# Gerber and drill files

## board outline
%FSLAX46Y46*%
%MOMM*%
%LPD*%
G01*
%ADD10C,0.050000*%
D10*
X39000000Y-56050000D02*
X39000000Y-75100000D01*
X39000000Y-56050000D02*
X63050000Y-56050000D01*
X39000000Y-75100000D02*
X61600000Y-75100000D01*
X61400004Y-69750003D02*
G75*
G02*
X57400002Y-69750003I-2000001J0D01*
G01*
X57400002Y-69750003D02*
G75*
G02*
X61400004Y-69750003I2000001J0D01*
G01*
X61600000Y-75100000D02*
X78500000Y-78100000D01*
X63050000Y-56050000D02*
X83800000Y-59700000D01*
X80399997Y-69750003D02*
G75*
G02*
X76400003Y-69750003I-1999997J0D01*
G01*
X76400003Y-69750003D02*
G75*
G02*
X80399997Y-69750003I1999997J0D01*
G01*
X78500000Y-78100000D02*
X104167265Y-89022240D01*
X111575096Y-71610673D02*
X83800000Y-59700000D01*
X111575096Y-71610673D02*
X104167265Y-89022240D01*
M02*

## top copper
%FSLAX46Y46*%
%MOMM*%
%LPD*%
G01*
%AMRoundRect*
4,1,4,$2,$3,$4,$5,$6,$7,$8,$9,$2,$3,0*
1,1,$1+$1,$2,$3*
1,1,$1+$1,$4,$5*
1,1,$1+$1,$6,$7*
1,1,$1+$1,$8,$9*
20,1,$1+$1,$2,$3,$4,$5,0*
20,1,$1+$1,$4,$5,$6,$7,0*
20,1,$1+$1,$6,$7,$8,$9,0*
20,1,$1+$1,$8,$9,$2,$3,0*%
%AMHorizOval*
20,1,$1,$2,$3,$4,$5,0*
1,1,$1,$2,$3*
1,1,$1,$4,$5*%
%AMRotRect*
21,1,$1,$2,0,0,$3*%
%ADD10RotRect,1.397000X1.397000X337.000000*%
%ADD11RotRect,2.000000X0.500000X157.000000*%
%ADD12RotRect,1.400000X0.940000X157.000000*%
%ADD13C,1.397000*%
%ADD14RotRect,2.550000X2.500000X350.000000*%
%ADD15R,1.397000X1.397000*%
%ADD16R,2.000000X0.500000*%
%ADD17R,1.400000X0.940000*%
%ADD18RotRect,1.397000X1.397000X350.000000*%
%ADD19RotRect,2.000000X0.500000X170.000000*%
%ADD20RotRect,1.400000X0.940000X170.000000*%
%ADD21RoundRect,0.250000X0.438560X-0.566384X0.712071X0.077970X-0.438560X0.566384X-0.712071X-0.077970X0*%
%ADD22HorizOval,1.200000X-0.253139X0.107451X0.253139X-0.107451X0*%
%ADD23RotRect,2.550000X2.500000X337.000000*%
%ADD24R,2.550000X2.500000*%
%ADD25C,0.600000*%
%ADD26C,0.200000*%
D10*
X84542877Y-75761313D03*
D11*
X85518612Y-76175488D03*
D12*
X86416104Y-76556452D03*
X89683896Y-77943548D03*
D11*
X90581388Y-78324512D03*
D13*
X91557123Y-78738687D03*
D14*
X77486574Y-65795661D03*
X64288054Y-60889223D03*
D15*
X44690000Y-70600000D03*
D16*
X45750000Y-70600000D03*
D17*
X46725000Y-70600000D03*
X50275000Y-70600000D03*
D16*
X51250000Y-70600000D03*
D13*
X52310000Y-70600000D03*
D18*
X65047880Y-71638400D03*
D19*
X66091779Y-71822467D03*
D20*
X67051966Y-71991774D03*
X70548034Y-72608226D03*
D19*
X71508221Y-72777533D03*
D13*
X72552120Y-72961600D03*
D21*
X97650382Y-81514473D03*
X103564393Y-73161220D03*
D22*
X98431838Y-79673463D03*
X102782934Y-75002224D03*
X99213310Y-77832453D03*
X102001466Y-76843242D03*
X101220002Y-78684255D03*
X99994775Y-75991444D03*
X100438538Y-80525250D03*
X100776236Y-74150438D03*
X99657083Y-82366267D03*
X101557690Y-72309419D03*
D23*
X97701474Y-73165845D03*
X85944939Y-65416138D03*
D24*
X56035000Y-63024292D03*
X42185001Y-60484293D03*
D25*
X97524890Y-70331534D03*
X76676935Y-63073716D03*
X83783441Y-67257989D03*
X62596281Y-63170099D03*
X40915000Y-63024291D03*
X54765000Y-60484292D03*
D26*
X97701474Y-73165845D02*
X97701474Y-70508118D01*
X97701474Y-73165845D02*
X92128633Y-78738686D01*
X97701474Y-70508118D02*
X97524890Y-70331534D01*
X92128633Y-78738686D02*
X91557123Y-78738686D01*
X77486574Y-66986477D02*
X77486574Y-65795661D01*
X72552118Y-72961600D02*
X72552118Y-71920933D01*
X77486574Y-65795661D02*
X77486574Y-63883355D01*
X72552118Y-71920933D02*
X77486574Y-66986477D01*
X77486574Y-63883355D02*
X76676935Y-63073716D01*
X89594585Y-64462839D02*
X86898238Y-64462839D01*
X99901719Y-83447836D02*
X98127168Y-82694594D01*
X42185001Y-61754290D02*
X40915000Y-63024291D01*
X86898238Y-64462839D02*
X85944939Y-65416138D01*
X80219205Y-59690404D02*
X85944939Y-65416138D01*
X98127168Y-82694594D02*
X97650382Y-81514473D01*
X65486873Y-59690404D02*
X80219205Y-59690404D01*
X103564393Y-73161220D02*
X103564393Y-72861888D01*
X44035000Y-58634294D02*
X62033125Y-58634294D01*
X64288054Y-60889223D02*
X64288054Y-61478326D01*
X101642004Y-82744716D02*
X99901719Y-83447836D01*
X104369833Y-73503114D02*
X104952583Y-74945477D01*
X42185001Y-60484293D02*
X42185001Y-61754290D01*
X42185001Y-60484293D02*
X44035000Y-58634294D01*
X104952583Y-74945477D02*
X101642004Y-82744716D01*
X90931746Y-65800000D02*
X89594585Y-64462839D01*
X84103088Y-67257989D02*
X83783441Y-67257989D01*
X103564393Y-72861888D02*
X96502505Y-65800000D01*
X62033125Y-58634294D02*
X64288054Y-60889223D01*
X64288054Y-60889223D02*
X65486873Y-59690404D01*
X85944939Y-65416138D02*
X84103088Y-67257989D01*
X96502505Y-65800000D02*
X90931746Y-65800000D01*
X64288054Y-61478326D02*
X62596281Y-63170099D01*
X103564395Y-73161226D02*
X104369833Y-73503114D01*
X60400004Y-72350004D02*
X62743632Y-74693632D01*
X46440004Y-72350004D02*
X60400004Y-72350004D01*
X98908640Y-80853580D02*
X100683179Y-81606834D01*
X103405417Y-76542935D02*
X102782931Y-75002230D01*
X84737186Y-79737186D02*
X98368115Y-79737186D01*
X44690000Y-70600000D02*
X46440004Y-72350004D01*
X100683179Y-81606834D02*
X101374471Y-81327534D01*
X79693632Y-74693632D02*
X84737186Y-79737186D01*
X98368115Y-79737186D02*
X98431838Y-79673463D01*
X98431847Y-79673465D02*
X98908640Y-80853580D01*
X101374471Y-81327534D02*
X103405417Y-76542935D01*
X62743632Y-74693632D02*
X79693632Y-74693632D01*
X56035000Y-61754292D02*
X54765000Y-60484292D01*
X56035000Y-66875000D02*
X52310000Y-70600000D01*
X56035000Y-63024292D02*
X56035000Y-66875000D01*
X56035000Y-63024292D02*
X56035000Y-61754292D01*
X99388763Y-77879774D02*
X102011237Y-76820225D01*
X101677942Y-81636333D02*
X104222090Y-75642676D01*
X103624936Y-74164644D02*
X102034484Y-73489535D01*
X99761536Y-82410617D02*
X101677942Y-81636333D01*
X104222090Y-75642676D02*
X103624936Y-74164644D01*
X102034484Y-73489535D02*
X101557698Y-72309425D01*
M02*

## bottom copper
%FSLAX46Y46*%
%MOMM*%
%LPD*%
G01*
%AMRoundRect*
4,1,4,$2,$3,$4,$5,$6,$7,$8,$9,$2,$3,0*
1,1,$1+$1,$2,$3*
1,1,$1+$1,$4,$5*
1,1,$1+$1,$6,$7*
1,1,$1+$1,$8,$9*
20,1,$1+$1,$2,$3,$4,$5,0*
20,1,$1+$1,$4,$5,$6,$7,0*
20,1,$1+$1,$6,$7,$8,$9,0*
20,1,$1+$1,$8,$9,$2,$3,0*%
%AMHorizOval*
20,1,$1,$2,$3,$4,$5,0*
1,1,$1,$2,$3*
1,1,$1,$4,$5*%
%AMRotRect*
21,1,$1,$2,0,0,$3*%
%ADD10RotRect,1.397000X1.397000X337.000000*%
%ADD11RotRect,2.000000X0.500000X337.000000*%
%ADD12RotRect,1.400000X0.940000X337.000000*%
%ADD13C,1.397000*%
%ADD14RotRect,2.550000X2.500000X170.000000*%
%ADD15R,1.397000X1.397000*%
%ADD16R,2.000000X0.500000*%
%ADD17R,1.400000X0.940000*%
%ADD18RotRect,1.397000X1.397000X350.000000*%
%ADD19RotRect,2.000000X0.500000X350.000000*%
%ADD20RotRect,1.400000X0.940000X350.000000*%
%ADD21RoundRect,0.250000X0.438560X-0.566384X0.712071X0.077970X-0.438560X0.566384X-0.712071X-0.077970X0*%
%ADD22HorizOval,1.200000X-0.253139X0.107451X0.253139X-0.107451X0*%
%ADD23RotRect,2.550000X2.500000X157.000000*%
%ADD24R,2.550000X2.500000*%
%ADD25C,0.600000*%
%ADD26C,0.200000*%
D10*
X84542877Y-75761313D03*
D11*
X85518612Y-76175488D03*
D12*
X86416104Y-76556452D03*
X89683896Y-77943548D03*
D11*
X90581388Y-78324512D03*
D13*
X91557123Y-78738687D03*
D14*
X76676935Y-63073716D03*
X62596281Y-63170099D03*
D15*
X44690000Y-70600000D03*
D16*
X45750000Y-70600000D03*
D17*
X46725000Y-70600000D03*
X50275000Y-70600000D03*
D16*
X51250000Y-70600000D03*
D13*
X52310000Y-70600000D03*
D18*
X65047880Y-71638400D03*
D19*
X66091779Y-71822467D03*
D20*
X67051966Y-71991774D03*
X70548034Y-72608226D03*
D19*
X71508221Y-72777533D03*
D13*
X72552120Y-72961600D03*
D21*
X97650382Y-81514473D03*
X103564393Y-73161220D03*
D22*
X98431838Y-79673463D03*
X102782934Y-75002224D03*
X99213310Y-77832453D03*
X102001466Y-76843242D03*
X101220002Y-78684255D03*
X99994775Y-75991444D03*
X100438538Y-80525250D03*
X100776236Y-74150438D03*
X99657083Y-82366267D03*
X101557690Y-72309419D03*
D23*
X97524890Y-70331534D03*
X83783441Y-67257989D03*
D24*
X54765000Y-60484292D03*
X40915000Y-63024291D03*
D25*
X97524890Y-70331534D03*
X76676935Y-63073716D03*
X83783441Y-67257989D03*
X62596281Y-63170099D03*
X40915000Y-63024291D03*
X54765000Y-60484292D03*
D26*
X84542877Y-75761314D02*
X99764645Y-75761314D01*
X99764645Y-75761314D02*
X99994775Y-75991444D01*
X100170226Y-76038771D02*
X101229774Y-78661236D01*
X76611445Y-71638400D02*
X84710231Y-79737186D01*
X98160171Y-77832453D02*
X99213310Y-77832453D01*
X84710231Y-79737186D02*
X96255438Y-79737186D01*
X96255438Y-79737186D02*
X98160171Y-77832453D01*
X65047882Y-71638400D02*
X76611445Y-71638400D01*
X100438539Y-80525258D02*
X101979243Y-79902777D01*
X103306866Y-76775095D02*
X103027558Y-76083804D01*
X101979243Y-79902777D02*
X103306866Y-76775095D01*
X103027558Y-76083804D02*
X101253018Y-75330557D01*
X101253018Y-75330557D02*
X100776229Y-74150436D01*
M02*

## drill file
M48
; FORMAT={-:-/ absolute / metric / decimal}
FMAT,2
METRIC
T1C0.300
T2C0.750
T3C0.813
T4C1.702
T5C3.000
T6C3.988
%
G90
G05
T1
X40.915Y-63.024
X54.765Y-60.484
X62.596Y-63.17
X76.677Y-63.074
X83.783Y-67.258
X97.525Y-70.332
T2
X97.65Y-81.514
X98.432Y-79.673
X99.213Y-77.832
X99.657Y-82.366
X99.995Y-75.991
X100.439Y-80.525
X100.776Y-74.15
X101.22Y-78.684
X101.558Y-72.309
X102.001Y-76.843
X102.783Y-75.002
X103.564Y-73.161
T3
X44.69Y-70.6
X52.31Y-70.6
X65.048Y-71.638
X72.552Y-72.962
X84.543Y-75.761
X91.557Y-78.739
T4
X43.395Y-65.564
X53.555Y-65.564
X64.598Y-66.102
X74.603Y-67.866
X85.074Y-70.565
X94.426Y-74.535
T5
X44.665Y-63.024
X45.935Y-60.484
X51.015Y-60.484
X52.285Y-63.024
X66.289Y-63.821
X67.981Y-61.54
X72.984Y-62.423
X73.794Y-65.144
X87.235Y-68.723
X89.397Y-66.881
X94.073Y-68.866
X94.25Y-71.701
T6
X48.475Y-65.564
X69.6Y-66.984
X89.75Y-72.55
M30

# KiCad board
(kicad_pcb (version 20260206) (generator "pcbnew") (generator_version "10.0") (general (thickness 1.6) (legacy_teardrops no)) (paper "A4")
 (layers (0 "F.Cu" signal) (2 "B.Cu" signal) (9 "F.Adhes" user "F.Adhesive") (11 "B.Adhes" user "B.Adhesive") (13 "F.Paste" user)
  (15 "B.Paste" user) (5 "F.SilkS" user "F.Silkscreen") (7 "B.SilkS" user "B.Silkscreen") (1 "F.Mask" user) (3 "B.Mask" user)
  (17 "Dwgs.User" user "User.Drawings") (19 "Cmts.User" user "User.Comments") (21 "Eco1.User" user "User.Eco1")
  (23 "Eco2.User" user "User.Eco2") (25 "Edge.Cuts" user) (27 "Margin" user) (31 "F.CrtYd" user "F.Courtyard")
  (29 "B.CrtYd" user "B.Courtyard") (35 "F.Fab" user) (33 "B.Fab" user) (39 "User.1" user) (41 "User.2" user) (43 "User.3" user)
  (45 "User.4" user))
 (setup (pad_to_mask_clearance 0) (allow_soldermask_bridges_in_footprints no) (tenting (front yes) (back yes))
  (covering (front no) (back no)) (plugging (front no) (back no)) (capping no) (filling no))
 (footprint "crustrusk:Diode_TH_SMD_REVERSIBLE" (layer "F.Cu") (at 88.05 77.25 -23)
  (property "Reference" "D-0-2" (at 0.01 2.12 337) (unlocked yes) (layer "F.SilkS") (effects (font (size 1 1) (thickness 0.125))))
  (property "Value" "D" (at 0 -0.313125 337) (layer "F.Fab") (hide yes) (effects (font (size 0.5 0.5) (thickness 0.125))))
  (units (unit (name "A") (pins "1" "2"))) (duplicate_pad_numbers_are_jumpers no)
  (pad "1" thru_hole rect (at -3.81 -0.000001 337) (size 1.397 1.397) (drill 0.8128) (layers "*.Cu" "*.Mask") (remove_unused_layers no)
   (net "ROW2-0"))
  (pad "1" smd rect (at -2.75 -0.000001 157) (size 2 0.5) (layers "F.Cu") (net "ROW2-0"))
  (pad "1" smd rect (at -2.75 -0.000001 337) (size 2 0.5) (layers "B.Cu") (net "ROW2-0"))
  (pad "1" smd rect (at -1.775 0 157) (size 1.4 0.94) (layers "F.Cu" "F.Mask" "F.Paste") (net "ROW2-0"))
  (pad "1" smd rect (at -1.775 0 337) (size 1.4 0.94) (layers "B.Cu" "B.Mask" "B.Paste") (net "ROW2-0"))
  (pad "2" smd rect (at 1.775 0 157) (size 1.4 0.94) (layers "F.Cu" "F.Mask" "F.Paste") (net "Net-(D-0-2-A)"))
  (pad "2" smd rect (at 1.775 0 337) (size 1.4 0.94) (layers "B.Cu" "B.Mask" "B.Paste") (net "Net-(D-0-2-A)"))
  (pad "2" smd rect (at 2.75 0.000001 157) (size 2 0.5) (layers "F.Cu") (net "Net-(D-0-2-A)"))
  (pad "2" smd rect (at 2.75 0.000001 337) (size 2 0.5) (layers "B.Cu") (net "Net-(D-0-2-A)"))
  (pad "2" thru_hole circle (at 3.81 0.000001 337) (size 1.397 1.397) (drill 0.8128) (layers "*.Cu" "*.Mask") (remove_unused_layers no)
   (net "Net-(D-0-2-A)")))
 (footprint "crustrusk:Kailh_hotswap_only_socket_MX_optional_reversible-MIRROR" (layer "F.Cu") (at 69.600361 66.984292 -10)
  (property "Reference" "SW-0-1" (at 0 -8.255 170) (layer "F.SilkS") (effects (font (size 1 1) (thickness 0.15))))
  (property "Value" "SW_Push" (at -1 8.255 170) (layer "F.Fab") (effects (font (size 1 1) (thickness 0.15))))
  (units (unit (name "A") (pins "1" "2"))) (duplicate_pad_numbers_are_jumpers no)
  (pad "" np_thru_hole circle (at -5.08 0 350) (size 1.7018 1.7018) (drill 1.7018) (layers "*.Cu" "*.Mask"))
  (pad "" np_thru_hole circle (at -3.81 -2.54 170) (size 3 3) (drill 3) (layers "*.Cu" "*.Mask"))
  (pad "" np_thru_hole circle (at -2.54 -5.079998 350) (size 3 3) (drill 3) (layers "*.Cu" "*.Mask"))
  (pad "" np_thru_hole circle (at 0 0 350) (size 3.9878 3.9878) (drill 3.9878) (layers "*.Cu" "*.Mask"))
  (pad "" np_thru_hole circle (at 2.540002 -5.080001 170) (size 3 3) (drill 3) (layers "*.Cu" "*.Mask"))
  (pad "" np_thru_hole circle (at 3.81 -2.54 350) (size 3 3) (drill 3) (layers "*.Cu" "*.Mask"))
  (pad "" np_thru_hole circle (at 5.08 0 350) (size 1.7018 1.7018) (drill 1.7018) (layers "*.Cu" "*.Mask"))
  (pad "1" smd rect (at 6.290001 -5.08 170) (size 2.55 2.5) (layers "B.Cu" "B.Mask" "B.Paste") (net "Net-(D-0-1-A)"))
  (pad "1" smd rect (at 7.56 -2.54 350) (size 2.55 2.5) (layers "F.Cu" "F.Mask" "F.Paste") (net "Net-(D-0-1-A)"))
  (pad "2" smd rect (at -7.56 -2.540001 170) (size 2.55 2.5) (layers "B.Cu" "B.Mask" "B.Paste") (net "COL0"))
  (pad "2" smd rect (at -6.289999 -5.079999 350) (size 2.55 2.5) (layers "F.Cu" "F.Mask" "F.Paste") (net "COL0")))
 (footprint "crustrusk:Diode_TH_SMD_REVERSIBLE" (layer "F.Cu") (at 48.5 70.6)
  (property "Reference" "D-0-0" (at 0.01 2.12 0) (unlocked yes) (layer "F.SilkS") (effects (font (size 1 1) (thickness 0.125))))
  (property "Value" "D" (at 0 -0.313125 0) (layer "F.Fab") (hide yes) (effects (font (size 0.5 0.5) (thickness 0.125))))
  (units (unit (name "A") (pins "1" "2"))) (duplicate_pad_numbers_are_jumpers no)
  (pad "1" thru_hole rect (at -3.81 0) (size 1.397 1.397) (drill 0.8128) (layers "*.Cu" "*.Mask") (remove_unused_layers no) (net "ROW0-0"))
  (pad "1" smd rect (at -2.75 0 180) (size 2 0.5) (layers "F.Cu") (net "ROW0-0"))
  (pad "1" smd rect (at -2.75 0) (size 2 0.5) (layers "B.Cu") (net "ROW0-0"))
  (pad "1" smd rect (at -1.775 0 180) (size 1.4 0.94) (layers "F.Cu" "F.Mask" "F.Paste") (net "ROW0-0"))
  (pad "1" smd rect (at -1.775 0) (size 1.4 0.94) (layers "B.Cu" "B.Mask" "B.Paste") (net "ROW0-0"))
  (pad "2" smd rect (at 1.775 0 180) (size 1.4 0.94) (layers "F.Cu" "F.Mask" "F.Paste") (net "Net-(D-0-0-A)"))
  (pad "2" smd rect (at 1.775 0) (size 1.4 0.94) (layers "B.Cu" "B.Mask" "B.Paste") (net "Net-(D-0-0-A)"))
  (pad "2" smd rect (at 2.75 0 180) (size 2 0.5) (layers "F.Cu") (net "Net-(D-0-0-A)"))
  (pad "2" smd rect (at 2.75 0) (size 2 0.5) (layers "B.Cu") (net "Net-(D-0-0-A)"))
  (pad "2" thru_hole circle (at 3.81 0) (size 1.397 1.397) (drill 0.8128) (layers "*.Cu" "*.Mask") (remove_unused_layers no)
   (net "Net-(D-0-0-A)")))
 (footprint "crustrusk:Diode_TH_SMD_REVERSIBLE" (layer "F.Cu") (at 68.8 72.3 -10)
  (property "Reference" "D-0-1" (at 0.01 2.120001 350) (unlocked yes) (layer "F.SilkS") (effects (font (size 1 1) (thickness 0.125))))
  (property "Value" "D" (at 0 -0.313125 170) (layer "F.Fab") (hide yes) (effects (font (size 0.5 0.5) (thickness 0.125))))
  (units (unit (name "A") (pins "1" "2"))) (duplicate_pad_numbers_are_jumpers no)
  (pad "1" thru_hole rect (at -3.810002 0 350) (size 1.397 1.397) (drill 0.8128) (layers "*.Cu" "*.Mask") (remove_unused_layers no)
   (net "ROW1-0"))
  (pad "1" smd rect (at -2.75 -0.000001 170) (size 2 0.5) (layers "F.Cu") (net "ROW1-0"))
  (pad "1" smd rect (at -2.75 -0.000001 350) (size 2 0.5) (layers "B.Cu") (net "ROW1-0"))
  (pad "1" smd rect (at -1.775 0 170) (size 1.4 0.94) (layers "F.Cu" "F.Mask" "F.Paste") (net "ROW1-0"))
  (pad "1" smd rect (at -1.775 0 350) (size 1.4 0.94) (layers "B.Cu" "B.Mask" "B.Paste") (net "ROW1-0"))
  (pad "2" smd rect (at 1.775 0 170) (size 1.4 0.94) (layers "F.Cu" "F.Mask" "F.Paste") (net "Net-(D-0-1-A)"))
  (pad "2" smd rect (at 1.775 0 350) (size 1.4 0.94) (layers "B.Cu" "B.Mask" "B.Paste") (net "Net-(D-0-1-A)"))
  (pad "2" smd rect (at 2.75 0.000001 170) (size 2 0.5) (layers "F.Cu") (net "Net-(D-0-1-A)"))
  (pad "2" smd rect (at 2.75 0.000001 350) (size 2 0.5) (layers "B.Cu") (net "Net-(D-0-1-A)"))
  (pad "2" thru_hole circle (at 3.810002 0 350) (size 1.397 1.397) (drill 0.8128) (layers "*.Cu" "*.Mask") (remove_unused_layers no)
   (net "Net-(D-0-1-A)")))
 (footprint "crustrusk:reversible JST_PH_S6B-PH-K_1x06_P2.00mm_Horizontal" (layer "F.Cu") (at 97.650382 81.514473 67)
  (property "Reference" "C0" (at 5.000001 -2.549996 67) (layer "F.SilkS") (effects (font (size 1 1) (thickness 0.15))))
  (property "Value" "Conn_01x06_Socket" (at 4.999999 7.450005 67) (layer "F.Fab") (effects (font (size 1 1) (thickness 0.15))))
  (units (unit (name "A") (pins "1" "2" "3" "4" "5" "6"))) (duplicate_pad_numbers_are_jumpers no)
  (pad "1" thru_hole roundrect (at 0 0 67) (size 1.2 1.75) (drill 0.75) (layers "*.Cu" "*.Mask") (remove_unused_layers no)
   (roundrect_rratio 0.208333) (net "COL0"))
  (pad "1" thru_hole roundrect (at 9.999998 2.18 67) (size 1.2 1.75) (drill 0.75) (layers "*.Cu" "*.Mask") (remove_unused_layers no)
   (roundrect_rratio 0.208333) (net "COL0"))
  (pad "2" thru_hole oval (at 1.999998 -0.000006 67) (size 1.2 1.75) (drill 0.75) (layers "*.Cu" "*.Mask") (remove_unused_layers no)
   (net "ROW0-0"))
  (pad "2" thru_hole oval (at 8.000005 2.180001 67) (size 1.2 1.75) (drill 0.75) (layers "*.Cu" "*.Mask") (remove_unused_layers no)
   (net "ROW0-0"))
  (pad "3" thru_hole oval (at 4.000002 0.000003 67) (size 1.2 1.75) (drill 0.75) (layers "*.Cu" "*.Mask") (remove_unused_layers no)
   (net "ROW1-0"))
  (pad "3" thru_hole oval (at 5.999995 2.179999 67) (size 1.2 1.75) (drill 0.75) (layers "*.Cu" "*.Mask") (remove_unused_layers no)
   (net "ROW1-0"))
  (pad "4" thru_hole oval (at 3.999991 2.179998 67) (size 1.2 1.75) (drill 0.75) (layers "*.Cu" "*.Mask") (remove_unused_layers no)
   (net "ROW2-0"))
  (pad "4" thru_hole oval (at 6.000002 0.000006 67) (size 1.2 1.75) (drill 0.75) (layers "*.Cu" "*.Mask") (remove_unused_layers no)
   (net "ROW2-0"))
  (pad "5" thru_hole oval (at 2.000004 2.179991 67) (size 1.2 1.75) (drill 0.75) (layers "*.Cu" "*.Mask") (remove_unused_layers no)
   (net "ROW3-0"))
  (pad "5" thru_hole oval (at 7.999998 0.000006 67) (size 1.2 1.75) (drill 0.75) (layers "*.Cu" "*.Mask") (remove_unused_layers no)
   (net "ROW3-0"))
  (pad "6" thru_hole oval (at 0 2.18 67) (size 1.2 1.75) (drill 0.75) (layers "*.Cu" "*.Mask") (remove_unused_layers no) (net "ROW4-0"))
  (pad "6" thru_hole oval (at 10.000004 -0.000005 67) (size 1.2 1.75) (drill 0.75) (layers "*.Cu" "*.Mask") (remove_unused_layers no)
   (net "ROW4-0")))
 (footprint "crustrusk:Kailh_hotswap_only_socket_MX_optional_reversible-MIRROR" (layer "F.Cu") (at 89.75 72.55 -23)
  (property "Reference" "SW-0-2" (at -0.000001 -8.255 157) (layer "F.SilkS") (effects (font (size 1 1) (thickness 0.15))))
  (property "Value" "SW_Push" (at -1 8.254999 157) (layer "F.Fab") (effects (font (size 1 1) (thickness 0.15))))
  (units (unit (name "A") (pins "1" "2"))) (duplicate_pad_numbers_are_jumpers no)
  (pad "" np_thru_hole circle (at -5.08 0 337) (size 1.7018 1.7018) (drill 1.7018) (layers "*.Cu" "*.Mask"))
  (pad "" np_thru_hole circle (at -3.81 -2.54 157) (size 3 3) (drill 3) (layers "*.Cu" "*.Mask"))
  (pad "" np_thru_hole circle (at -2.54 -5.079998 337) (size 3 3) (drill 3) (layers "*.Cu" "*.Mask"))
  (pad "" np_thru_hole circle (at 0 0 337) (size 3.9878 3.9878) (drill 3.9878) (layers "*.Cu" "*.Mask"))
  (pad "" np_thru_hole circle (at 2.540002 -5.080001 157) (size 3 3) (drill 3) (layers "*.Cu" "*.Mask"))
  (pad "" np_thru_hole circle (at 3.81 -2.54 337) (size 3 3) (drill 3) (layers "*.Cu" "*.Mask"))
  (pad "" np_thru_hole circle (at 5.08 0 337) (size 1.7018 1.7018) (drill 1.7018) (layers "*.Cu" "*.Mask"))
  (pad "1" smd rect (at 6.29 -5.08 157) (size 2.55 2.5) (layers "B.Cu" "B.Mask" "B.Paste") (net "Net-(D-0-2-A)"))
  (pad "1" smd rect (at 7.56 -2.54 337) (size 2.55 2.5) (layers "F.Cu" "F.Mask" "F.Paste") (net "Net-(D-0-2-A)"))
  (pad "2" smd rect (at -7.56 -2.540001 157) (size 2.55 2.5) (layers "B.Cu" "B.Mask" "B.Paste") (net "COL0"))
  (pad "2" smd rect (at -6.289999 -5.079999 337) (size 2.55 2.5) (layers "F.Cu" "F.Mask" "F.Paste") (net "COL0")))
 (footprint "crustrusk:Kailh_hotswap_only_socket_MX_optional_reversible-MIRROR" (layer "F.Cu") (at 48.475 65.564292)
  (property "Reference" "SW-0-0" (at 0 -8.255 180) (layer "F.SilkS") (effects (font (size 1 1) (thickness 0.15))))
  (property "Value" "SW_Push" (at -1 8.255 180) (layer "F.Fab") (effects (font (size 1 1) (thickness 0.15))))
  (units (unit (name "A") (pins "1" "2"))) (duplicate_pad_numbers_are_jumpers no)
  (pad "" np_thru_hole circle (at -5.08 0) (size 1.7018 1.7018) (drill 1.7018) (layers "*.Cu" "*.Mask"))
  (pad "" np_thru_hole circle (at -3.81 -2.54 180) (size 3 3) (drill 3) (layers "*.Cu" "*.Mask"))
  (pad "" np_thru_hole circle (at -2.54 -5.079998) (size 3 3) (drill 3) (layers "*.Cu" "*.Mask"))
  (pad "" np_thru_hole circle (at 0 0) (size 3.9878 3.9878) (drill 3.9878) (layers "*.Cu" "*.Mask"))
  (pad "" np_thru_hole circle (at 2.540002 -5.080001 180) (size 3 3) (drill 3) (layers "*.Cu" "*.Mask"))
  (pad "" np_thru_hole circle (at 3.81 -2.54) (size 3 3) (drill 3) (layers "*.Cu" "*.Mask"))
  (pad "" np_thru_hole circle (at 5.08 0) (size 1.7018 1.7018) (drill 1.7018) (layers "*.Cu" "*.Mask"))
  (pad "1" smd rect (at 6.29 -5.08 180) (size 2.55 2.5) (layers "B.Cu" "B.Mask" "B.Paste") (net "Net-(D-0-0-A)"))
  (pad "1" smd rect (at 7.56 -2.54) (size 2.55 2.5) (layers "F.Cu" "F.Mask" "F.Paste") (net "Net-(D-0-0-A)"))
  (pad "2" smd rect (at -7.56 -2.540001 180) (size 2.55 2.5) (layers "B.Cu" "B.Mask" "B.Paste") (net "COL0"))
  (pad "2" smd rect (at -6.289999 -5.079999) (size 2.55 2.5) (layers "F.Cu" "F.Mask" "F.Paste") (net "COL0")))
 (gr_line (start 39 56.05) (end 39 75.1) (stroke (width 0.05) (type default)) (layer "Edge.Cuts"))
 (gr_line (start 39 56.05) (end 63.05 56.05) (stroke (width 0.05) (type default)) (layer "Edge.Cuts"))
 (gr_line (start 39 75.1) (end 61.6 75.1) (stroke (width 0.05) (type default)) (layer "Edge.Cuts"))
 (gr_circle (center 59.400003 69.750003) (end 57.400002 69.750003) (stroke (width 0.05) (type default)) (fill no) (layer "Edge.Cuts"))
 (gr_line (start 61.6 75.1) (end 78.5 78.1) (stroke (width 0.05) (type default)) (layer "Edge.Cuts"))
 (gr_line (start 63.05 56.05) (end 83.8 59.7) (stroke (width 0.05) (type default)) (layer "Edge.Cuts"))
 (gr_circle (center 78.4 69.750003) (end 76.400003 69.750003) (stroke (width 0.05) (type default)) (fill no) (layer "Edge.Cuts"))
 (gr_line (start 78.5 78.1) (end 104.167265 89.02224) (stroke (width 0.05) (type default)) (layer "Edge.Cuts"))
 (gr_line (start 111.575096 71.610673) (end 83.8 59.7) (stroke (width 0.05) (type default)) (layer "Edge.Cuts"))
 (gr_line (start 111.575096 71.610673) (end 104.167265 89.02224) (stroke (width 0.05) (type default)) (layer "Edge.Cuts"))
 (segment (start 84.542877 75.761314) (end 99.764645 75.761314) (width 0.2) (layer "B.Cu") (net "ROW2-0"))
 (segment (start 99.764645 75.761314) (end 99.994775 75.991444) (width 0.2) (layer "B.Cu") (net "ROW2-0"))
 (segment (start 100.170226 76.038771) (end 101.229774 78.661236) (width 0.2) (layer "B.Cu") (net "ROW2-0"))
 (segment (start 97.701474 73.165845) (end 97.701474 70.508118) (width 0.2) (layer "F.Cu") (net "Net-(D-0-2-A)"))
 (segment (start 97.701474 73.165845) (end 92.128633 78.738686) (width 0.2) (layer "F.Cu") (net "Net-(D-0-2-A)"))
 (segment (start 97.701474 70.508118) (end 97.52489 70.331534) (width 0.2) (layer "F.Cu") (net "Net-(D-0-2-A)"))
 (segment (start 92.128633 78.738686) (end 91.557123 78.738686) (width 0.2) (layer "F.Cu") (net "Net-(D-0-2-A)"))
 (via (at 97.52489 70.331534) (size 0.6) (drill 0.3) (layers "F.Cu" "B.Cu") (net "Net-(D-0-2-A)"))
 (segment (start 77.486574 66.986477) (end 77.486574 65.795661) (width 0.2) (layer "F.Cu") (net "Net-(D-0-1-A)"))
 (segment (start 72.552118 72.9616) (end 72.552118 71.920933) (width 0.2) (layer "F.Cu") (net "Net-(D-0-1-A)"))
 (segment (start 77.486574 65.795661) (end 77.486574 63.883355) (width 0.2) (layer "F.Cu") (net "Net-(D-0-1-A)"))
 (segment (start 72.552118 71.920933) (end 77.486574 66.986477) (width 0.2) (layer "F.Cu") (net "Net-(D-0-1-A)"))
 (segment (start 77.486574 63.883355) (end 76.676935 63.073716) (width 0.2) (layer "F.Cu") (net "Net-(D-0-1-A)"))
 (via (at 76.676935 63.073716) (size 0.6) (drill 0.3) (layers "F.Cu" "B.Cu") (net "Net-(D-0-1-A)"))
 (segment (start 89.594585 64.462839) (end 86.898238 64.462839) (width 0.2) (layer "F.Cu") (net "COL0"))
 (segment (start 99.901719 83.447836) (end 98.127168 82.694594) (width 0.2) (layer "F.Cu") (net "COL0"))
 (segment (start 42.185001 61.75429) (end 40.915 63.024291) (width 0.2) (layer "F.Cu") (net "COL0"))
 (segment (start 86.898238 64.462839) (end 85.944939 65.416138) (width 0.2) (layer "F.Cu") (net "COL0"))
 (segment (start 80.219205 59.690404) (end 85.944939 65.416138) (width 0.2) (layer "F.Cu") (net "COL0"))
 (segment (start 98.127168 82.694594) (end 97.650382 81.514473) (width 0.2) (layer "F.Cu") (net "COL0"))
 (segment (start 65.486873 59.690404) (end 80.219205 59.690404) (width 0.2) (layer "F.Cu") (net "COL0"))
 (segment (start 103.564393 73.16122) (end 103.564393 72.861888) (width 0.2) (layer "F.Cu") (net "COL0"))
 (segment (start 44.035 58.634294) (end 62.033125 58.634294) (width 0.2) (layer "F.Cu") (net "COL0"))
 (segment (start 64.288054 60.889223) (end 64.288054 61.478326) (width 0.2) (layer "F.Cu") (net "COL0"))
 (segment (start 101.642004 82.744716) (end 99.901719 83.447836) (width 0.2) (layer "F.Cu") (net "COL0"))
 (segment (start 104.369833 73.503114) (end 104.952583 74.945477) (width 0.2) (layer "F.Cu") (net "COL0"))
 (segment (start 42.185001 60.484293) (end 42.185001 61.75429) (width 0.2) (layer "F.Cu") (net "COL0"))
 (segment (start 42.185001 60.484293) (end 44.035 58.634294) (width 0.2) (layer "F.Cu") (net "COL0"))
 (segment (start 104.952583 74.945477) (end 101.642004 82.744716) (width 0.2) (layer "F.Cu") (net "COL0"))
 (segment (start 90.931746 65.8) (end 89.594585 64.462839) (width 0.2) (layer "F.Cu") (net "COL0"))
 (segment (start 84.103088 67.257989) (end 83.783441 67.257989) (width 0.2) (layer "F.Cu") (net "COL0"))
 (segment (start 103.564393 72.861888) (end 96.502505 65.8) (width 0.2) (layer "F.Cu") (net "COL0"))
 (segment (start 62.033125 58.634294) (end 64.288054 60.889223) (width 0.2) (layer "F.Cu") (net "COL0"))
 (segment (start 64.288054 60.889223) (end 65.486873 59.690404) (width 0.2) (layer "F.Cu") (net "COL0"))
 (segment (start 85.944939 65.416138) (end 84.103088 67.257989) (width 0.2) (layer "F.Cu") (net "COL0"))
 (segment (start 96.502505 65.8) (end 90.931746 65.8) (width 0.2) (layer "F.Cu") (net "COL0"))
 (segment (start 64.288054 61.478326) (end 62.596281 63.170099) (width 0.2) (layer "F.Cu") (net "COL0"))
 (segment (start 103.564395 73.161226) (end 104.369833 73.503114) (width 0.2) (layer "F.Cu") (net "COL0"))
 (via (at 83.783441 67.257989) (size 0.6) (drill 0.3) (layers "F.Cu" "B.Cu") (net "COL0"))
 (via (at 62.596281 63.170099) (size 0.6) (drill 0.3) (layers "F.Cu" "B.Cu") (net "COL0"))
 (via (at 40.915 63.024291) (size 0.6) (drill 0.3) (layers "F.Cu" "B.Cu") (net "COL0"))
 (segment (start 60.400004 72.350004) (end 62.743632 74.693632) (width 0.2) (layer "F.Cu") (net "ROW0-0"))
 (segment (start 46.440004 72.350004) (end 60.400004 72.350004) (width 0.2) (layer "F.Cu") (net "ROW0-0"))
 (segment (start 98.90864 80.85358) (end 100.683179 81.606834) (width 0.2) (layer "F.Cu") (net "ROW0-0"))
 (segment (start 103.405417 76.542935) (end 102.782931 75.00223) (width 0.2) (layer "F.Cu") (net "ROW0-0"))
 (segment (start 84.737186 79.737186) (end 98.368115 79.737186) (width 0.2) (layer "F.Cu") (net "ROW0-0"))
 (segment (start 44.69 70.6) (end 46.440004 72.350004) (width 0.2) (layer "F.Cu") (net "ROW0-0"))
 (segment (start 100.683179 81.606834) (end 101.374471 81.327534) (width 0.2) (layer "F.Cu") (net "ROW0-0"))
 (segment (start 79.693632 74.693632) (end 84.737186 79.737186) (width 0.2) (layer "F.Cu") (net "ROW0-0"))
 (segment (start 98.368115 79.737186) (end 98.431838 79.673463) (width 0.2) (layer "F.Cu") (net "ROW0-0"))
 (segment (start 98.431847 79.673465) (end 98.90864 80.85358) (width 0.2) (layer "F.Cu") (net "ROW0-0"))
 (segment (start 101.374471 81.327534) (end 103.405417 76.542935) (width 0.2) (layer "F.Cu") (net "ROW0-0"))
 (segment (start 62.743632 74.693632) (end 79.693632 74.693632) (width 0.2) (layer "F.Cu") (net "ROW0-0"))
 (segment (start 56.035 61.754292) (end 54.765 60.484292) (width 0.2) (layer "F.Cu") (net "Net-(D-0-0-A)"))
 (segment (start 56.035 66.875) (end 52.31 70.6) (width 0.2) (layer "F.Cu") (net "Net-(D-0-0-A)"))
 (segment (start 56.035 63.024292) (end 56.035 66.875) (width 0.2) (layer "F.Cu") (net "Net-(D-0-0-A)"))
 (segment (start 56.035 63.024292) (end 56.035 61.754292) (width 0.2) (layer "F.Cu") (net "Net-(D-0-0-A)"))
 (via (at 54.765 60.484292) (size 0.6) (drill 0.3) (layers "F.Cu" "B.Cu") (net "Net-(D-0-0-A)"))
 (segment (start 99.388763 77.879774) (end 102.011237 76.820225) (width 0.2) (layer "F.Cu") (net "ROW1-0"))
 (segment (start 76.611445 71.6384) (end 84.710231 79.737186) (width 0.2) (layer "B.Cu") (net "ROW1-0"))
 (segment (start 98.160171 77.832453) (end 99.21331 77.832453) (width 0.2) (layer "B.Cu") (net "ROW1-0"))
 (segment (start 84.710231 79.737186) (end 96.255438 79.737186) (width 0.2) (layer "B.Cu") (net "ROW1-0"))
 (segment (start 96.255438 79.737186) (end 98.160171 77.832453) (width 0.2) (layer "B.Cu") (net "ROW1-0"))
 (segment (start 65.047882 71.6384) (end 76.611445 71.6384) (width 0.2) (layer "B.Cu") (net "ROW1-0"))
 (segment (start 100.438539 80.525258) (end 101.979243 79.902777) (width 0.2) (layer "B.Cu") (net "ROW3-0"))
 (segment (start 103.306866 76.775095) (end 103.027558 76.083804) (width 0.2) (layer "B.Cu") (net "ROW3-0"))
 (segment (start 101.979243 79.902777) (end 103.306866 76.775095) (width 0.2) (layer "B.Cu") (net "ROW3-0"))
 (segment (start 103.027558 76.083804) (end 101.253018 75.330557) (width 0.2) (layer "B.Cu") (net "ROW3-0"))
 (segment (start 101.253018 75.330557) (end 100.776229 74.150436) (width 0.2) (layer "B.Cu") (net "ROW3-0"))
 (segment (start 101.677942 81.636333) (end 104.22209 75.642676) (width 0.2) (layer "F.Cu") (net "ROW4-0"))
 (segment (start 103.624936 74.164644) (end 102.034484 73.489535) (width 0.2) (layer "F.Cu") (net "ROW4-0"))
 (segment (start 99.761536 82.410617) (end 101.677942 81.636333) (width 0.2) (layer "F.Cu") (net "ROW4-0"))
 (segment (start 104.22209 75.642676) (end 103.624936 74.164644) (width 0.2) (layer "F.Cu") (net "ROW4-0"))
 (segment (start 102.034484 73.489535) (end 101.557698 72.309425) (width 0.2) (layer "F.Cu") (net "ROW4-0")))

